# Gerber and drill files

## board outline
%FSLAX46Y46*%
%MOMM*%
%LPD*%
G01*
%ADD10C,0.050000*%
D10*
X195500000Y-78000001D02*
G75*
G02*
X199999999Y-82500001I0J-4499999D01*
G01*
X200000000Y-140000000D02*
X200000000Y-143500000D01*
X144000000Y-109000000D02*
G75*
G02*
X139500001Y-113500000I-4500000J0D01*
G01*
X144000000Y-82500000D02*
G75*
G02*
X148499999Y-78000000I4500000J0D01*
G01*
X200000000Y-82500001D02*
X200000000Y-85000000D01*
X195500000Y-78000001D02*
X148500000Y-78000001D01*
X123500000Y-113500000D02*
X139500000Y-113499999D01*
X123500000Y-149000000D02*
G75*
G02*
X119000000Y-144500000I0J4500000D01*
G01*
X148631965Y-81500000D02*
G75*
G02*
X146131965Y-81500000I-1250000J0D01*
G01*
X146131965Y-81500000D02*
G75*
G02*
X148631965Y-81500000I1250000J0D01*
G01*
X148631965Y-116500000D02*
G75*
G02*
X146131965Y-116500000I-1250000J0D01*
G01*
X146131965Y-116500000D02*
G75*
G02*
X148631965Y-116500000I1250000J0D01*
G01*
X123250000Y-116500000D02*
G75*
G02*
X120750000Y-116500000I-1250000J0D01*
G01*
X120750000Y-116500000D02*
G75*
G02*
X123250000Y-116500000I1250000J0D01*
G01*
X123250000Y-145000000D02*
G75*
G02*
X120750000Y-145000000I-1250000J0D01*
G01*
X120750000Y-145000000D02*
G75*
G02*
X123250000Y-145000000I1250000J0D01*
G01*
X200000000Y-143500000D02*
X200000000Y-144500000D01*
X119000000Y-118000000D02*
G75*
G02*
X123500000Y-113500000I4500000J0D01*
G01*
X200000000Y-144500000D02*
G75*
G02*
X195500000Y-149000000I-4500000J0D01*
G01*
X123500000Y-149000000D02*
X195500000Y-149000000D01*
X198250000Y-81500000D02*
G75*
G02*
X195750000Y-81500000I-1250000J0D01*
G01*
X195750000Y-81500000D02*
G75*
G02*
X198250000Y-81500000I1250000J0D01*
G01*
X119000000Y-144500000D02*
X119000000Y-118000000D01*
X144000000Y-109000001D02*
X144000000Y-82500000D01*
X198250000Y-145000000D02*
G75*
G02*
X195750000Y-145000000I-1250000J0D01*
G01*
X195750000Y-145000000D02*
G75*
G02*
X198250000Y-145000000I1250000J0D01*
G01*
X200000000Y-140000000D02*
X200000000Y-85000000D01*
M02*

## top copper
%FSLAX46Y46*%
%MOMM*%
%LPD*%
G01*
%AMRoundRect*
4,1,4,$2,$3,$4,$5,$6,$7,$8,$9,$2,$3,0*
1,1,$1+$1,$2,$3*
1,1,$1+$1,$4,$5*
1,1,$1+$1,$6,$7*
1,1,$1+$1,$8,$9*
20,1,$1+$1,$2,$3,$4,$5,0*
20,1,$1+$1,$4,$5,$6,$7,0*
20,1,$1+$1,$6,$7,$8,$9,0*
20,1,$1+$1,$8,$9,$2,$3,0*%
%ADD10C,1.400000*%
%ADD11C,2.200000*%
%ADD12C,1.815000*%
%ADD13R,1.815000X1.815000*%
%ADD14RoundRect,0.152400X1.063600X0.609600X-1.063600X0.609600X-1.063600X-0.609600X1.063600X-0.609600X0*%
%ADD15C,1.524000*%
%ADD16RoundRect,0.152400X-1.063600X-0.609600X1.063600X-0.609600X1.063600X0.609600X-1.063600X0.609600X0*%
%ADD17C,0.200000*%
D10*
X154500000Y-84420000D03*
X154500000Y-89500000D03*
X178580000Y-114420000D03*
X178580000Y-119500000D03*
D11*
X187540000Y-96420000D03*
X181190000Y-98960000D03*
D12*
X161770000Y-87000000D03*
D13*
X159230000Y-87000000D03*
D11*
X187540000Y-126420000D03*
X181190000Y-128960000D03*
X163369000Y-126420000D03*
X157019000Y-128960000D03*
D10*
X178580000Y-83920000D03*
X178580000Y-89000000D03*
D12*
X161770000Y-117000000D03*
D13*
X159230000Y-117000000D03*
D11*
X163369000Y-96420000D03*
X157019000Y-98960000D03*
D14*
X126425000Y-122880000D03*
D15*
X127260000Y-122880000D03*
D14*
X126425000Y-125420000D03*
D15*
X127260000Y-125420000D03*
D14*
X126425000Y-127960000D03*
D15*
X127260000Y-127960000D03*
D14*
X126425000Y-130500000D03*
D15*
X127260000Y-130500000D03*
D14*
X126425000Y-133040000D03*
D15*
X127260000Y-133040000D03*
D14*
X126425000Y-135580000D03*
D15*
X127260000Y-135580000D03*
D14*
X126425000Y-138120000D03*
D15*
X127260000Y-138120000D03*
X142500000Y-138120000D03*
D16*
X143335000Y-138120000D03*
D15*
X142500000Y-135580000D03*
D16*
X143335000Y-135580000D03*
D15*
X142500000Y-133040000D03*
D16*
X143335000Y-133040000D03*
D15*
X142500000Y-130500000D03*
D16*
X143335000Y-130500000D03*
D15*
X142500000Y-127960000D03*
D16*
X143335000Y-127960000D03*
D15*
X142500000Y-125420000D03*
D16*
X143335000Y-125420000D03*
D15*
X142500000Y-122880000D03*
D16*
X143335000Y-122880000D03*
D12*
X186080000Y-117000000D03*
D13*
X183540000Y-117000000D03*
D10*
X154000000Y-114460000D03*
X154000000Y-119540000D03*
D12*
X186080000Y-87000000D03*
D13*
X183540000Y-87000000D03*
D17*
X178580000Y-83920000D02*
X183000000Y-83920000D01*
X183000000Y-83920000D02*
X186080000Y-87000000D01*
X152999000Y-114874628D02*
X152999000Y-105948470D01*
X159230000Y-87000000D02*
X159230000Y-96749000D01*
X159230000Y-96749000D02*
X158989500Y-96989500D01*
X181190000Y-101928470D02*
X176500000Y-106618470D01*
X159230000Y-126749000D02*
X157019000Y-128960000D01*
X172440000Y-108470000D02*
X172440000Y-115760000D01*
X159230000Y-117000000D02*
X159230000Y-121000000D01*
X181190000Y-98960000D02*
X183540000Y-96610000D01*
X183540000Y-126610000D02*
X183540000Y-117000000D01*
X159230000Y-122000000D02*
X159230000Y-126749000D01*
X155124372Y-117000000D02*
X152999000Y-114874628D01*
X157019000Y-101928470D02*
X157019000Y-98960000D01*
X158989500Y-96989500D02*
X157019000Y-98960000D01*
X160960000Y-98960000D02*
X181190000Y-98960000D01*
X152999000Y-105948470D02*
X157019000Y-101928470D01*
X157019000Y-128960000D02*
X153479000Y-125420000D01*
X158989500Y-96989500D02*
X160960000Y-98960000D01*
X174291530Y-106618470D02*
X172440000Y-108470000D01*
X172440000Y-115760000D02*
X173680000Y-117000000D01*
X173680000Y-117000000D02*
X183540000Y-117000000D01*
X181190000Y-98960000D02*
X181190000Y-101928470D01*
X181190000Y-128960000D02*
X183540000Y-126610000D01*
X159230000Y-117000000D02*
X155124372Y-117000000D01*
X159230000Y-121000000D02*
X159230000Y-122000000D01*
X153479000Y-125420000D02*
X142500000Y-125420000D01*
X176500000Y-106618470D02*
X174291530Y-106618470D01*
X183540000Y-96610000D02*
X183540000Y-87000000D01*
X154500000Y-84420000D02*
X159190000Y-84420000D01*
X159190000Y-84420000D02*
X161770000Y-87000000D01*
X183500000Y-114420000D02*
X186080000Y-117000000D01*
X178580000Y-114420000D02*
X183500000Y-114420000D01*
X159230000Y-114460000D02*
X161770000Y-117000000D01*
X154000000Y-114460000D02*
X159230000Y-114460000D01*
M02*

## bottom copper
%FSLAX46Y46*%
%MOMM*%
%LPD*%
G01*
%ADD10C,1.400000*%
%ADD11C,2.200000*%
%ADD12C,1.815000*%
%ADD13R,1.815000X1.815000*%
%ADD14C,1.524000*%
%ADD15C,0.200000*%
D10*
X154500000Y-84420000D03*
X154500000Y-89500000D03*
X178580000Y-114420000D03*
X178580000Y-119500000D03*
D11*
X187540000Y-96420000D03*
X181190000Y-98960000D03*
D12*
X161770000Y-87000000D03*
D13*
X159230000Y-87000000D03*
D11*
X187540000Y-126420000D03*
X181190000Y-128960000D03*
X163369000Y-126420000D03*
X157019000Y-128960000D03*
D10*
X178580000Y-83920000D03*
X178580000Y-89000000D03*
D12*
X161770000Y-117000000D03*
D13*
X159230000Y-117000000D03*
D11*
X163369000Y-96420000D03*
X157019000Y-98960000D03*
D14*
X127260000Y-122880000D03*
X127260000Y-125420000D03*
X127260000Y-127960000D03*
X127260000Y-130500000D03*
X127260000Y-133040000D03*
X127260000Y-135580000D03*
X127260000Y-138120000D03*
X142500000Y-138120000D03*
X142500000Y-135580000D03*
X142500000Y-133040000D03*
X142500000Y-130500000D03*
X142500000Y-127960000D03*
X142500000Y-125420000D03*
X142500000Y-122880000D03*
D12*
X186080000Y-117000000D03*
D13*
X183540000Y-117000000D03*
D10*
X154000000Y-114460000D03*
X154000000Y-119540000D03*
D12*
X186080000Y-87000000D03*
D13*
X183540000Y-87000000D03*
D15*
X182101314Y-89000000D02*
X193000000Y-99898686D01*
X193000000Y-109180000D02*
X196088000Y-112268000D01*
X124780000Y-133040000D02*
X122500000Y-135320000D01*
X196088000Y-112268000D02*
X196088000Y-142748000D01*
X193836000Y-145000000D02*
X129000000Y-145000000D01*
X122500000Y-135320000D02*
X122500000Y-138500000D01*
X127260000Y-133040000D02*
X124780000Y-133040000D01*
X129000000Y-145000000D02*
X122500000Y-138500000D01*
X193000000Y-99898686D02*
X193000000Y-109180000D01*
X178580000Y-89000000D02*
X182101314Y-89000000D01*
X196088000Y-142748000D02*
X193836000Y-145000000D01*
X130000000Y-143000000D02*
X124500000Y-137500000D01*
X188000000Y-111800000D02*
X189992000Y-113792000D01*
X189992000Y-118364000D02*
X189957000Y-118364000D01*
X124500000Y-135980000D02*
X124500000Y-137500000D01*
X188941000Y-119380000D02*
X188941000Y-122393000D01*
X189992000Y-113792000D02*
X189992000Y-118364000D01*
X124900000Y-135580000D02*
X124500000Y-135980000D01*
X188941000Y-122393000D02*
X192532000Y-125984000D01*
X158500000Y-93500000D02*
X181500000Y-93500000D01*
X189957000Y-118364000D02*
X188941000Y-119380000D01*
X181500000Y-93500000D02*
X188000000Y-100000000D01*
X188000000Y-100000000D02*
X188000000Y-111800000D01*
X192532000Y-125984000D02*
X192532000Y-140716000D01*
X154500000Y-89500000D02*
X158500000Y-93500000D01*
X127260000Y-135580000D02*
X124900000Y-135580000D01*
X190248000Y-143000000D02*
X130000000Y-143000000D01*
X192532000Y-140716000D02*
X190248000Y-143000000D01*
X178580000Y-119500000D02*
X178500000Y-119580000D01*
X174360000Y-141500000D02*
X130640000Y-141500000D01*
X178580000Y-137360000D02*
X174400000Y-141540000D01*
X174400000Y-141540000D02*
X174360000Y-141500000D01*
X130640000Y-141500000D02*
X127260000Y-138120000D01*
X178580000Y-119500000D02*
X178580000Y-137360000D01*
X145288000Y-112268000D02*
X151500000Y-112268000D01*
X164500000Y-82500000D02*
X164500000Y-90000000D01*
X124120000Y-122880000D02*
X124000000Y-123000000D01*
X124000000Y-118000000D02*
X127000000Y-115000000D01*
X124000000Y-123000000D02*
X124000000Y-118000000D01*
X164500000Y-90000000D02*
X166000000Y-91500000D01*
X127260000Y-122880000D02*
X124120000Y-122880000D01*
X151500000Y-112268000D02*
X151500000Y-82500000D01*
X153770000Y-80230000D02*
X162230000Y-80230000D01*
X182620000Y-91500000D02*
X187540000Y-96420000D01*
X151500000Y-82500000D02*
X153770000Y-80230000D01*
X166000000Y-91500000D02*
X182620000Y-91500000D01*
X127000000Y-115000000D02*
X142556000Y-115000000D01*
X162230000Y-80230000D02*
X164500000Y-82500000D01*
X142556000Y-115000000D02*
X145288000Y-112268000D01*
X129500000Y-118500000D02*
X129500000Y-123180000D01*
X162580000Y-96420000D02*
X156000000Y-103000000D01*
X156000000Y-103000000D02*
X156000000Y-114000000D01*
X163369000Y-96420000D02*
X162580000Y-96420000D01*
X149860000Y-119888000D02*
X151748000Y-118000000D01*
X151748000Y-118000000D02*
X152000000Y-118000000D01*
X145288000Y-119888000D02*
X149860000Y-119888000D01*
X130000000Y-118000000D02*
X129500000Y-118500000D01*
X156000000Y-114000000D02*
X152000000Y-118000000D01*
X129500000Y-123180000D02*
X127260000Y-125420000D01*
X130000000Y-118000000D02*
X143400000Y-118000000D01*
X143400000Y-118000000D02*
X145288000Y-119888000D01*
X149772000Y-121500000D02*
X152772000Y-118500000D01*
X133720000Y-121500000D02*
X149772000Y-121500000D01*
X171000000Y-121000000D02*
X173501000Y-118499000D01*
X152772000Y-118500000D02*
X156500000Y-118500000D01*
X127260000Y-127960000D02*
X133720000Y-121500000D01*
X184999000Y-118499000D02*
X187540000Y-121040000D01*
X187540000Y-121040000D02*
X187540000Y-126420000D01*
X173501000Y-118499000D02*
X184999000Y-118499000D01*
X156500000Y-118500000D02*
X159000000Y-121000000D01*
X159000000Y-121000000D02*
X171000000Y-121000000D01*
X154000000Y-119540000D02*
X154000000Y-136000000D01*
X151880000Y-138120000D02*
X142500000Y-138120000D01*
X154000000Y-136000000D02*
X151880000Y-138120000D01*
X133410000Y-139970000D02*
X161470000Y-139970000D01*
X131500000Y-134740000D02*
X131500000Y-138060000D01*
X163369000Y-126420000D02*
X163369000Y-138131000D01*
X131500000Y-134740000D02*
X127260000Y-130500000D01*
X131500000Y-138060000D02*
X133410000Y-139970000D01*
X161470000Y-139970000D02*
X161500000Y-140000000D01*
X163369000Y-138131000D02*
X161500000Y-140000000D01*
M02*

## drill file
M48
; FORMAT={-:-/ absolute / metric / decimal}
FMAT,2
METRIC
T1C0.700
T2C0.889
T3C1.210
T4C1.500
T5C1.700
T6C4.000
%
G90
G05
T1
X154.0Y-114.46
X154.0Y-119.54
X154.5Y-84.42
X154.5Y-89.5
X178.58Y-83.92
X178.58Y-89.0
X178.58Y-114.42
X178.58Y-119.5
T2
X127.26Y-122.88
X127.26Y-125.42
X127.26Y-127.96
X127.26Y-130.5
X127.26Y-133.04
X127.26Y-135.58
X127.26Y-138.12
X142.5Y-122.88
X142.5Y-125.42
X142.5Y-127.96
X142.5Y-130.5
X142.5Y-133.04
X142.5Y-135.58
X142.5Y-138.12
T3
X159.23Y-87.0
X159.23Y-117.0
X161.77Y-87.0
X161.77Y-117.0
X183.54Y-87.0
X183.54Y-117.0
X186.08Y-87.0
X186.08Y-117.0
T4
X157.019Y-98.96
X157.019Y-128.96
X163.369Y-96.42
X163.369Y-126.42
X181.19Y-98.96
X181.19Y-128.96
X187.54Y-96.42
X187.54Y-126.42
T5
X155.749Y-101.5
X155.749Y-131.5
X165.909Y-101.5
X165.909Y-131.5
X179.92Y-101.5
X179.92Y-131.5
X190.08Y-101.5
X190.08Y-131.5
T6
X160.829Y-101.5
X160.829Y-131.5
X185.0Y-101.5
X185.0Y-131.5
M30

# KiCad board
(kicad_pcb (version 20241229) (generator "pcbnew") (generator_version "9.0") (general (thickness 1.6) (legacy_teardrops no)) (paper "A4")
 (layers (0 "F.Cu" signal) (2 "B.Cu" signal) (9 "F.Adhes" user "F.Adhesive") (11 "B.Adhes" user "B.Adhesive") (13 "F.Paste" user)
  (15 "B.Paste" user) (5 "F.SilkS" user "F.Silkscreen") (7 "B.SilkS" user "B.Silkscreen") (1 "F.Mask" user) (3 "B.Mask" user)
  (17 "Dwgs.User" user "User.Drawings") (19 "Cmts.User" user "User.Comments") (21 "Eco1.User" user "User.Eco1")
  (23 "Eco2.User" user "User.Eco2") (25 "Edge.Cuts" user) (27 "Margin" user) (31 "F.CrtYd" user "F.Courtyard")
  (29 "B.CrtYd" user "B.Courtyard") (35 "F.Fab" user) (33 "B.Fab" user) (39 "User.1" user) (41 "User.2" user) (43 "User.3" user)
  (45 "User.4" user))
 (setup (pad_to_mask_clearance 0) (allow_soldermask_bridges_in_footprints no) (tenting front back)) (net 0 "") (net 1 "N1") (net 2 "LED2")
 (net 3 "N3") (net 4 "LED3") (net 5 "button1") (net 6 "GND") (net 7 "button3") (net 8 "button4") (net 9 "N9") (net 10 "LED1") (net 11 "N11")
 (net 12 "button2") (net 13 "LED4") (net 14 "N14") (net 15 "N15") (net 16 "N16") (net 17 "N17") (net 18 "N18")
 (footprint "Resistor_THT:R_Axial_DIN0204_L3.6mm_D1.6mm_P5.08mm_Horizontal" (layer "F.Cu") (at 154.5 84.42 -90)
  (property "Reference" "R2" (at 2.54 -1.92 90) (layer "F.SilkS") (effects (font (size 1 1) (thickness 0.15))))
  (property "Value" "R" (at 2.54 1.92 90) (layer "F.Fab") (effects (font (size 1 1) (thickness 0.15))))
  (pad "1" thru_hole circle (at 0 0 270) (size 1.4 1.4) (drill 0.7) (layers "*.Cu" "*.Mask") (remove_unused_layers no) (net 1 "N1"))
  (pad "2" thru_hole circle (at 5.08 0 270) (size 1.4 1.4) (drill 0.7) (layers "*.Cu" "*.Mask") (remove_unused_layers no) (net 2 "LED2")))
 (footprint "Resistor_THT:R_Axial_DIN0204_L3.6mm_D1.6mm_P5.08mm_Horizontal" (layer "F.Cu") (at 178.58 114.42 -90)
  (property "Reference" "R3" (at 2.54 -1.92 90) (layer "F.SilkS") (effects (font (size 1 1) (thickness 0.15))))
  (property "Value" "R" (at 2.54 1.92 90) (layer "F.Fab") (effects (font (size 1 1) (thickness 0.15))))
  (pad "1" thru_hole circle (at 0 0 270) (size 1.4 1.4) (drill 0.7) (layers "*.Cu" "*.Mask") (remove_unused_layers no) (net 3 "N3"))
  (pad "2" thru_hole circle (at 5.08 0 270) (size 1.4 1.4) (drill 0.7) (layers "*.Cu" "*.Mask") (remove_unused_layers no) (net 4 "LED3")))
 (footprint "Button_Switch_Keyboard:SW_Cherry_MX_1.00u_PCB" (layer "F.Cu") (at 187.54 96.42)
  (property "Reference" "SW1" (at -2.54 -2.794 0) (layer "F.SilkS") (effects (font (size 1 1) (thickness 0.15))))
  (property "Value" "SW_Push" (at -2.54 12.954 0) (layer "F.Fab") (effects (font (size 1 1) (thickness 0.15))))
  (pad "" np_thru_hole circle (at -7.62 5.08) (size 1.7 1.7) (drill 1.7) (layers "*.Cu" "*.Mask"))
  (pad "" np_thru_hole circle (at -2.54 5.08) (size 4 4) (drill 4) (layers "*.Cu" "*.Mask"))
  (pad "" np_thru_hole circle (at 2.54 5.08) (size 1.7 1.7) (drill 1.7) (layers "*.Cu" "*.Mask"))
  (pad "1" thru_hole circle (at 0 0) (size 2.2 2.2) (drill 1.5) (layers "*.Cu" "*.Mask") (remove_unused_layers no) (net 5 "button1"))
  (pad "2" thru_hole circle (at -6.35 2.54) (size 2.2 2.2) (drill 1.5) (layers "*.Cu" "*.Mask") (remove_unused_layers no) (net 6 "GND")))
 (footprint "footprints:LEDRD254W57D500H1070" (layer "F.Cu") (at 160.5 87)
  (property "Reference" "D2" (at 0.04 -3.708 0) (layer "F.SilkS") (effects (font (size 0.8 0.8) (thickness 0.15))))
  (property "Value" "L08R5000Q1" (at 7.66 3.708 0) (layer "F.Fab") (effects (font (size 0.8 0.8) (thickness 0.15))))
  (pad "A" thru_hole circle (at 1.27 0) (size 1.815 1.815) (drill 1.21) (layers "*.Cu" "*.Mask") (remove_unused_layers no) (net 1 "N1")
   (solder_mask_margin 0.102))
  (pad "C" thru_hole rect (at -1.27 0) (size 1.815 1.815) (drill 1.21) (layers "*.Cu" "*.Mask") (remove_unused_layers no) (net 6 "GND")
   (solder_mask_margin 0.102)))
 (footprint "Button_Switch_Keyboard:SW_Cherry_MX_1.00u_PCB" (layer "F.Cu") (at 187.54 126.42)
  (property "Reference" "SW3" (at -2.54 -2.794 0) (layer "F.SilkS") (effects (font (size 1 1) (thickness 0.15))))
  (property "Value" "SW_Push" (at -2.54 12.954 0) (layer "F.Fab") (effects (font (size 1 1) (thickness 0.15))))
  (pad "" np_thru_hole circle (at -7.62 5.08) (size 1.7 1.7) (drill 1.7) (layers "*.Cu" "*.Mask"))
  (pad "" np_thru_hole circle (at -2.54 5.08) (size 4 4) (drill 4) (layers "*.Cu" "*.Mask"))
  (pad "" np_thru_hole circle (at 2.54 5.08) (size 1.7 1.7) (drill 1.7) (layers "*.Cu" "*.Mask"))
  (pad "1" thru_hole circle (at 0 0) (size 2.2 2.2) (drill 1.5) (layers "*.Cu" "*.Mask") (remove_unused_layers no) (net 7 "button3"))
  (pad "2" thru_hole circle (at -6.35 2.54) (size 2.2 2.2) (drill 1.5) (layers "*.Cu" "*.Mask") (remove_unused_layers no) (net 6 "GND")))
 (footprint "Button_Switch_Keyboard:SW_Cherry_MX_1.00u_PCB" (layer "F.Cu") (at 163.369 126.42)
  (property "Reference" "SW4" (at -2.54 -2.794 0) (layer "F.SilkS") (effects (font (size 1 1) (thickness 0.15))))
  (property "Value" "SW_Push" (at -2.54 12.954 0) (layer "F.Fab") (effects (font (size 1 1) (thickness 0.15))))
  (pad "" np_thru_hole circle (at -7.62 5.08) (size 1.7 1.7) (drill 1.7) (layers "*.Cu" "*.Mask"))
  (pad "" np_thru_hole circle (at -2.54 5.08) (size 4 4) (drill 4) (layers "*.Cu" "*.Mask"))
  (pad "" np_thru_hole circle (at 2.54 5.08) (size 1.7 1.7) (drill 1.7) (layers "*.Cu" "*.Mask"))
  (pad "1" thru_hole circle (at 0 0) (size 2.2 2.2) (drill 1.5) (layers "*.Cu" "*.Mask") (remove_unused_layers no) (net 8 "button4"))
  (pad "2" thru_hole circle (at -6.35 2.54) (size 2.2 2.2) (drill 1.5) (layers "*.Cu" "*.Mask") (remove_unused_layers no) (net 6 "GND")))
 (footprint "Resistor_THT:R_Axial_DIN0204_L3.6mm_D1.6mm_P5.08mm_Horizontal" (layer "F.Cu") (at 178.58 83.92 -90)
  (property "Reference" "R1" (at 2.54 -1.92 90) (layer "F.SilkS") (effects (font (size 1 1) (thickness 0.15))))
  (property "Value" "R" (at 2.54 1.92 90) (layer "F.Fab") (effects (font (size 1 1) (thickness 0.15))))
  (pad "1" thru_hole circle (at 0 0 270) (size 1.4 1.4) (drill 0.7) (layers "*.Cu" "*.Mask") (remove_unused_layers no) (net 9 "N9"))
  (pad "2" thru_hole circle (at 5.08 0 270) (size 1.4 1.4) (drill 0.7) (layers "*.Cu" "*.Mask") (remove_unused_layers no) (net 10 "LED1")))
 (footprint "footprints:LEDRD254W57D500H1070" (layer "F.Cu") (at 160.5 117)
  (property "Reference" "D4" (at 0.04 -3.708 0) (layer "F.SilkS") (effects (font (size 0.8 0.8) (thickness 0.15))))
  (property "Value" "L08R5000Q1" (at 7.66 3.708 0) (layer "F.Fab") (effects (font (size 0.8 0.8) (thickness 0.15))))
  (pad "A" thru_hole circle (at 1.27 0) (size 1.815 1.815) (drill 1.21) (layers "*.Cu" "*.Mask") (remove_unused_layers no) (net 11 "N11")
   (solder_mask_margin 0.102))
  (pad "C" thru_hole rect (at -1.27 0) (size 1.815 1.815) (drill 1.21) (layers "*.Cu" "*.Mask") (remove_unused_layers no) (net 6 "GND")
   (solder_mask_margin 0.102)))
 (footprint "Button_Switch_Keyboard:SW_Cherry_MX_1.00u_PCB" (layer "F.Cu") (at 163.369 96.42)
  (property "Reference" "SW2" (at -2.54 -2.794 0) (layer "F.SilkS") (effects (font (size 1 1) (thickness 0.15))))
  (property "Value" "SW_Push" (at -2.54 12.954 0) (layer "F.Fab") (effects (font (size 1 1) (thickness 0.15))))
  (pad "" np_thru_hole circle (at -7.62 5.08) (size 1.7 1.7) (drill 1.7) (layers "*.Cu" "*.Mask"))
  (pad "" np_thru_hole circle (at -2.54 5.08) (size 4 4) (drill 4) (layers "*.Cu" "*.Mask"))
  (pad "" np_thru_hole circle (at 2.54 5.08) (size 1.7 1.7) (drill 1.7) (layers "*.Cu" "*.Mask"))
  (pad "1" thru_hole circle (at 0 0) (size 2.2 2.2) (drill 1.5) (layers "*.Cu" "*.Mask") (remove_unused_layers no) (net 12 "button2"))
  (pad "2" thru_hole circle (at -6.35 2.54) (size 2.2 2.2) (drill 1.5) (layers "*.Cu" "*.Mask") (remove_unused_layers no) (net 6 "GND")))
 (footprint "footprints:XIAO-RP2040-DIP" (layer "F.Cu") (at 134.88 130.5)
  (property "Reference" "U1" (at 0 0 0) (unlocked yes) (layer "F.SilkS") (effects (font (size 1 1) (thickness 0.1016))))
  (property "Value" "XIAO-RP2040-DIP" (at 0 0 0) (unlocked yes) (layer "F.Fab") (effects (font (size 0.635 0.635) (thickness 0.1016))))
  (pad "1" smd roundrect (at -8.455 -7.62 180) (size 2.432 1.524) (layers "F.Cu" "F.Mask") (roundrect_rratio 0.1) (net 5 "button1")
   (thermal_bridge_angle 45))
  (pad "1" thru_hole circle (at -7.62 -7.62 180) (size 1.524 1.524) (drill 0.889) (layers "*.Cu" "*.Mask") (remove_unused_layers no)
   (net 5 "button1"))
  (pad "2" smd roundrect (at -8.455 -5.08 180) (size 2.432 1.524) (layers "F.Cu" "F.Mask") (roundrect_rratio 0.1) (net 12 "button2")
   (thermal_bridge_angle 45))
  (pad "2" thru_hole circle (at -7.62 -5.08 180) (size 1.524 1.524) (drill 0.889) (layers "*.Cu" "*.Mask") (remove_unused_layers no)
   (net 12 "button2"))
  (pad "3" smd roundrect (at -8.455 -2.54 180) (size 2.432 1.524) (layers "F.Cu" "F.Mask") (roundrect_rratio 0.1) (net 7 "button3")
   (thermal_bridge_angle 45))
  (pad "3" thru_hole circle (at -7.62 -2.54 180) (size 1.524 1.524) (drill 0.889) (layers "*.Cu" "*.Mask") (remove_unused_layers no)
   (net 7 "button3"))
  (pad "4" smd roundrect (at -8.455 0 180) (size 2.432 1.524) (layers "F.Cu" "F.Mask") (roundrect_rratio 0.1) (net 8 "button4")
   (thermal_bridge_angle 45))
  (pad "4" thru_hole circle (at -7.62 0 180) (size 1.524 1.524) (drill 0.889) (layers "*.Cu" "*.Mask") (remove_unused_layers no)
   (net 8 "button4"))
  (pad "5" smd roundrect (at -8.455 2.54 180) (size 2.432 1.524) (layers "F.Cu" "F.Mask") (roundrect_rratio 0.1) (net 10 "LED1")
   (thermal_bridge_angle 45))
  (pad "5" thru_hole circle (at -7.62 2.54 180) (size 1.524 1.524) (drill 0.889) (layers "*.Cu" "*.Mask") (remove_unused_layers no)
   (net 10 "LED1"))
  (pad "6" smd roundrect (at -8.455 5.08 180) (size 2.432 1.524) (layers "F.Cu" "F.Mask") (roundrect_rratio 0.1) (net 2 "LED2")
   (thermal_bridge_angle 45))
  (pad "6" thru_hole circle (at -7.62 5.08 180) (size 1.524 1.524) (drill 0.889) (layers "*.Cu" "*.Mask") (remove_unused_layers no)
   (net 2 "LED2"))
  (pad "7" smd roundrect (at -8.455 7.62 180) (size 2.432 1.524) (layers "F.Cu" "F.Mask") (roundrect_rratio 0.1) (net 4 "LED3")
   (thermal_bridge_angle 45))
  (pad "7" thru_hole circle (at -7.62 7.62 180) (size 1.524 1.524) (drill 0.889) (layers "*.Cu" "*.Mask") (remove_unused_layers no)
   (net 4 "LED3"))
  (pad "8" thru_hole circle (at 7.62 7.62) (size 1.524 1.524) (drill 0.889) (layers "*.Cu" "*.Mask") (remove_unused_layers no)
   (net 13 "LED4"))
  (pad "8" smd roundrect (at 8.455 7.62) (size 2.432 1.524) (layers "F.Cu" "F.Mask") (roundrect_rratio 0.1) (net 13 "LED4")
   (thermal_bridge_angle 45))
  (pad "9" thru_hole circle (at 7.62 5.08) (size 1.524 1.524) (drill 0.889) (layers "*.Cu" "*.Mask") (remove_unused_layers no)
   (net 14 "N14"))
  (pad "9" smd roundrect (at 8.455 5.08) (size 2.432 1.524) (layers "F.Cu" "F.Mask") (roundrect_rratio 0.1) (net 14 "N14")
   (thermal_bridge_angle 45))
  (pad "10" thru_hole circle (at 7.62 2.54) (size 1.524 1.524) (drill 0.889) (layers "*.Cu" "*.Mask") (remove_unused_layers no)
   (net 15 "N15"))
  (pad "10" smd roundrect (at 8.455 2.54) (size 2.432 1.524) (layers "F.Cu" "F.Mask") (roundrect_rratio 0.1) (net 15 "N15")
   (thermal_bridge_angle 45))
  (pad "11" thru_hole circle (at 7.62 0) (size 1.524 1.524) (drill 0.889) (layers "*.Cu" "*.Mask") (remove_unused_layers no) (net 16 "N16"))
  (pad "11" smd roundrect (at 8.455 0) (size 2.432 1.524) (layers "F.Cu" "F.Mask") (roundrect_rratio 0.1) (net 16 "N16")
   (thermal_bridge_angle 45))
  (pad "12" thru_hole circle (at 7.62 -2.54) (size 1.524 1.524) (drill 0.889) (layers "*.Cu" "*.Mask") (remove_unused_layers no)
   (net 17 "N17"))
  (pad "12" smd roundrect (at 8.455 -2.54) (size 2.432 1.524) (layers "F.Cu" "F.Mask") (roundrect_rratio 0.1) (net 17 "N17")
   (thermal_bridge_angle 45))
  (pad "13" thru_hole circle (at 7.62 -5.08) (size 1.524 1.524) (drill 0.889) (layers "*.Cu" "*.Mask") (remove_unused_layers no)
   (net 6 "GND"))
  (pad "13" smd roundrect (at 8.455 -5.08) (size 2.432 1.524) (layers "F.Cu" "F.Mask") (roundrect_rratio 0.1) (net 6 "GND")
   (thermal_bridge_angle 45))
  (pad "14" thru_hole circle (at 7.62 -7.62) (size 1.524 1.524) (drill 0.889) (layers "*.Cu" "*.Mask") (remove_unused_layers no)
   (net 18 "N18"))
  (pad "14" smd roundrect (at 8.455 -7.62) (size 2.432 1.524) (layers "F.Cu" "F.Mask") (roundrect_rratio 0.1) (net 18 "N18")
   (thermal_bridge_angle 45)))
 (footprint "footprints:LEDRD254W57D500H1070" (layer "F.Cu") (at 184.81 117)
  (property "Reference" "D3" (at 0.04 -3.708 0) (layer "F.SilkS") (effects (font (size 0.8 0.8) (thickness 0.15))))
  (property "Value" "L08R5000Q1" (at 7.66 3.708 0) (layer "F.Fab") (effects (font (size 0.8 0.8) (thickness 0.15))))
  (pad "A" thru_hole circle (at 1.27 0) (size 1.815 1.815) (drill 1.21) (layers "*.Cu" "*.Mask") (remove_unused_layers no) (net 3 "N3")
   (solder_mask_margin 0.102))
  (pad "C" thru_hole rect (at -1.27 0) (size 1.815 1.815) (drill 1.21) (layers "*.Cu" "*.Mask") (remove_unused_layers no) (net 6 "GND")
   (solder_mask_margin 0.102)))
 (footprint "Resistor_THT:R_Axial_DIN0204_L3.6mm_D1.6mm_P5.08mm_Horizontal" (layer "F.Cu") (at 154 114.46 -90)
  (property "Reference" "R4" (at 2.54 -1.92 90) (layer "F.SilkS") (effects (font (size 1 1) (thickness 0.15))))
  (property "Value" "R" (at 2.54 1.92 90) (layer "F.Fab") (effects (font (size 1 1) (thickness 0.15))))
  (pad "1" thru_hole circle (at 0 0 270) (size 1.4 1.4) (drill 0.7) (layers "*.Cu" "*.Mask") (remove_unused_layers no) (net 11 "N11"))
  (pad "2" thru_hole circle (at 5.08 0 270) (size 1.4 1.4) (drill 0.7) (layers "*.Cu" "*.Mask") (remove_unused_layers no) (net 13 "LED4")))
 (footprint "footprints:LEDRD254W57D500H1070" (layer "F.Cu") (at 184.81 87)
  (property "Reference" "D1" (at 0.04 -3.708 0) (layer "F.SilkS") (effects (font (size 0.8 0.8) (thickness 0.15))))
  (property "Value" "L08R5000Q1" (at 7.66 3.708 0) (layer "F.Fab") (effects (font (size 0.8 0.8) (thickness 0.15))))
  (pad "A" thru_hole circle (at 1.27 0) (size 1.815 1.815) (drill 1.21) (layers "*.Cu" "*.Mask") (remove_unused_layers no) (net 9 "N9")
   (solder_mask_margin 0.102))
  (pad "C" thru_hole rect (at -1.27 0) (size 1.815 1.815) (drill 1.21) (layers "*.Cu" "*.Mask") (remove_unused_layers no) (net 6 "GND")
   (solder_mask_margin 0.102)))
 (gr_arc (start 195.5 78.000001) (mid 198.681981 79.31802) (end 200 82.500001) (stroke (width 0.05) (type default)) (layer "Edge.Cuts"))
 (gr_line (start 200 140) (end 200 143.5) (stroke (width 0.05) (type default)) (layer "Edge.Cuts"))
 (gr_arc (start 144 109) (mid 142.681982 112.181986) (end 139.500001 113.499999) (stroke (width 0.05) (type default)) (layer "Edge.Cuts"))
 (gr_arc (start 144 82.5) (mid 145.31802 79.318026) (end 148.499999 78.000001) (stroke (width 0.05) (type default)) (layer "Edge.Cuts"))
 (gr_line (start 200 82.500001) (end 200 85) (stroke (width 0.05) (type default)) (layer "Edge.Cuts"))
 (gr_line (start 195.5 78.000001) (end 148.5 78.000001) (stroke (width 0.05) (type default)) (layer "Edge.Cuts"))
 (gr_line (start 123.5 113.5) (end 139.5 113.499999) (stroke (width 0.05) (type default)) (layer "Edge.Cuts"))
 (gr_arc (start 123.5 149) (mid 120.318019 147.681981) (end 119 144.5) (stroke (width 0.05) (type default)) (layer "Edge.Cuts"))
 (gr_circle (center 147.381965 81.5) (end 148.631965 81.5) (stroke (width 0.05) (type solid)) (fill no) (layer "Edge.Cuts"))
 (gr_circle (center 147.381965 116.5) (end 148.631965 116.5) (stroke (width 0.05) (type solid)) (fill no) (layer "Edge.Cuts"))
 (gr_circle (center 122 116.5) (end 123.25 116.5) (stroke (width 0.05) (type solid)) (fill no) (layer "Edge.Cuts"))
 (gr_circle (center 122 145) (end 123.25 145) (stroke (width 0.05) (type solid)) (fill no) (layer "Edge.Cuts"))
 (gr_line (start 200 143.5) (end 200 144.5) (stroke (width 0.05) (type default)) (layer "Edge.Cuts"))
 (gr_arc (start 119 118) (mid 120.31802 114.81802) (end 123.5 113.5) (stroke (width 0.05) (type default)) (layer "Edge.Cuts"))
 (gr_arc (start 200 144.5) (mid 198.681981 147.681981) (end 195.5 149) (stroke (width 0.05) (type default)) (layer "Edge.Cuts"))
 (gr_line (start 123.5 149) (end 195.5 149) (stroke (width 0.05) (type default)) (layer "Edge.Cuts"))
 (gr_circle (center 197 81.5) (end 198.25 81.5) (stroke (width 0.05) (type solid)) (fill no) (layer "Edge.Cuts"))
 (gr_line (start 119 144.5) (end 119 118) (stroke (width 0.05) (type default)) (layer "Edge.Cuts"))
 (gr_line (start 144 109.000001) (end 144 82.5) (stroke (width 0.05) (type default)) (layer "Edge.Cuts"))
 (gr_circle (center 197 145) (end 198.25 145) (stroke (width 0.05) (type solid)) (fill no) (layer "Edge.Cuts"))
 (gr_line (start 200 140) (end 200 85) (stroke (width 0.05) (type solid)) (layer "Edge.Cuts"))
 (segment (start 178.58 83.92) (end 183 83.92) (width 0.2) (layer "F.Cu") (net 9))
 (segment (start 183 83.92) (end 186.08 87) (width 0.2) (layer "F.Cu") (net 9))
 (segment (start 152.999 114.874628) (end 152.999 105.94847) (width 0.2) (layer "F.Cu") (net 6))
 (segment (start 159.23 87) (end 159.23 96.749) (width 0.2) (layer "F.Cu") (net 6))
 (segment (start 159.23 96.749) (end 158.9895 96.9895) (width 0.2) (layer "F.Cu") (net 6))
 (segment (start 181.19 101.92847) (end 176.5 106.61847) (width 0.2) (layer "F.Cu") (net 6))
 (segment (start 159.23 126.749) (end 157.019 128.96) (width 0.2) (layer "F.Cu") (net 6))
 (segment (start 172.44 108.47) (end 172.44 115.76) (width 0.2) (layer "F.Cu") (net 6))
 (segment (start 159.23 117) (end 159.23 121) (width 0.2) (layer "F.Cu") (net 6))
 (segment (start 181.19 98.96) (end 183.54 96.61) (width 0.2) (layer "F.Cu") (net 6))
 (segment (start 183.54 126.61) (end 183.54 117) (width 0.2) (layer "F.Cu") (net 6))
 (segment (start 159.23 122) (end 159.23 126.749) (width 0.2) (layer "F.Cu") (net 6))
 (segment (start 155.124372 117) (end 152.999 114.874628) (width 0.2) (layer "F.Cu") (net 6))
 (segment (start 157.019 101.92847) (end 157.019 98.96) (width 0.2) (layer "F.Cu") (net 6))
 (segment (start 158.9895 96.9895) (end 157.019 98.96) (width 0.2) (layer "F.Cu") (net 6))
 (segment (start 160.96 98.96) (end 181.19 98.96) (width 0.2) (layer "F.Cu") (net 6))
 (segment (start 152.999 105.94847) (end 157.019 101.92847) (width 0.2) (layer "F.Cu") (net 6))
 (segment (start 157.019 128.96) (end 153.479 125.42) (width 0.2) (layer "F.Cu") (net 6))
 (segment (start 158.9895 96.9895) (end 160.96 98.96) (width 0.2) (layer "F.Cu") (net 6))
 (segment (start 174.29153 106.61847) (end 172.44 108.47) (width 0.2) (layer "F.Cu") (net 6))
 (segment (start 172.44 115.76) (end 173.68 117) (width 0.2) (layer "F.Cu") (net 6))
 (segment (start 173.68 117) (end 183.54 117) (width 0.2) (layer "F.Cu") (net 6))
 (segment (start 181.19 98.96) (end 181.19 101.92847) (width 0.2) (layer "F.Cu") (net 6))
 (segment (start 181.19 128.96) (end 183.54 126.61) (width 0.2) (layer "F.Cu") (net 6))
 (segment (start 159.23 117) (end 155.124372 117) (width 0.2) (layer "F.Cu") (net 6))
 (segment (start 159.23 121) (end 159.23 122) (width 0.2) (layer "F.Cu") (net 6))
 (segment (start 153.479 125.42) (end 142.5 125.42) (width 0.2) (layer "F.Cu") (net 6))
 (segment (start 176.5 106.61847) (end 174.29153 106.61847) (width 0.2) (layer "F.Cu") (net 6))
 (segment (start 183.54 96.61) (end 183.54 87) (width 0.2) (layer "F.Cu") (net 6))
 (segment (start 154.5 84.42) (end 159.19 84.42) (width 0.2) (layer "F.Cu") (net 1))
 (segment (start 159.19 84.42) (end 161.77 87) (width 0.2) (layer "F.Cu") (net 1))
 (segment (start 183.5 114.42) (end 186.08 117) (width 0.2) (layer "F.Cu") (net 3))
 (segment (start 178.58 114.42) (end 183.5 114.42) (width 0.2) (layer "F.Cu") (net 3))
 (segment (start 182.101314 89) (end 193 99.898686) (width 0.2) (layer "B.Cu") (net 10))
 (segment (start 193 109.18) (end 196.088 112.268) (width 0.2) (layer "B.Cu") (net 10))
 (segment (start 124.78 133.04) (end 122.5 135.32) (width 0.2) (layer "B.Cu") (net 10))
 (segment (start 196.088 112.268) (end 196.088 142.748) (width 0.2) (layer "B.Cu") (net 10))
 (segment (start 193.836 145) (end 129 145) (width 0.2) (layer "B.Cu") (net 10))
 (segment (start 122.5 135.32) (end 122.5 138.5) (width 0.2) (layer "B.Cu") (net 10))
 (segment (start 127.26 133.04) (end 124.78 133.04) (width 0.2) (layer "B.Cu") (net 10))
 (segment (start 129 145) (end 122.5 138.5) (width 0.2) (layer "B.Cu") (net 10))
 (segment (start 193 99.898686) (end 193 109.18) (width 0.2) (layer "B.Cu") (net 10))
 (segment (start 178.58 89) (end 182.101314 89) (width 0.2) (layer "B.Cu") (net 10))
 (segment (start 196.088 142.748) (end 193.836 145) (width 0.2) (layer "B.Cu") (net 10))
 (segment (start 130 143) (end 124.5 137.5) (width 0.2) (layer "B.Cu") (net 2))
 (segment (start 188 111.8) (end 189.992 113.792) (width 0.2) (layer "B.Cu") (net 2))
 (segment (start 189.992 118.364) (end 189.957 118.364) (width 0.2) (layer "B.Cu") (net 2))
 (segment (start 124.5 135.98) (end 124.5 137.5) (width 0.2) (layer "B.Cu") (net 2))
 (segment (start 188.941 119.38) (end 188.941 122.393) (width 0.2) (layer "B.Cu") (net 2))
 (segment (start 189.992 113.792) (end 189.992 118.364) (width 0.2) (layer "B.Cu") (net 2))
 (segment (start 124.9 135.58) (end 124.5 135.98) (width 0.2) (layer "B.Cu") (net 2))
 (segment (start 188.941 122.393) (end 192.532 125.984) (width 0.2) (layer "B.Cu") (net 2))
 (segment (start 158.5 93.5) (end 181.5 93.5) (width 0.2) (layer "B.Cu") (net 2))
 (segment (start 189.957 118.364) (end 188.941 119.38) (width 0.2) (layer "B.Cu") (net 2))
 (segment (start 181.5 93.5) (end 188 100) (width 0.2) (layer "B.Cu") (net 2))
 (segment (start 188 100) (end 188 111.8) (width 0.2) (layer "B.Cu") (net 2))
 (segment (start 192.532 125.984) (end 192.532 140.716) (width 0.2) (layer "B.Cu") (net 2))
 (segment (start 154.5 89.5) (end 158.5 93.5) (width 0.2) (layer "B.Cu") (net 2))
 (segment (start 127.26 135.58) (end 124.9 135.58) (width 0.2) (layer "B.Cu") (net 2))
 (segment (start 190.248 143) (end 130 143) (width 0.2) (layer "B.Cu") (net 2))
 (segment (start 192.532 140.716) (end 190.248 143) (width 0.2) (layer "B.Cu") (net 2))
 (segment (start 178.58 119.5) (end 178.5 119.58) (width 0.2) (layer "B.Cu") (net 4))
 (segment (start 174.36 141.5) (end 130.64 141.5) (width 0.2) (layer "B.Cu") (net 4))
 (segment (start 178.58 137.36) (end 174.4 141.54) (width 0.2) (layer "B.Cu") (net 4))
 (segment (start 174.4 141.54) (end 174.36 141.5) (width 0.2) (layer "B.Cu") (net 4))
 (segment (start 130.64 141.5) (end 127.26 138.12) (width 0.2) (layer "B.Cu") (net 4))
 (segment (start 178.58 119.5) (end 178.58 137.36) (width 0.2) (layer "B.Cu") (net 4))
 (segment (start 145.288 112.268) (end 151.5 112.268) (width 0.2) (layer "B.Cu") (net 5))
 (segment (start 164.5 82.5) (end 164.5 90) (width 0.2) (layer "B.Cu") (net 5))
 (segment (start 124.12 122.88) (end 124 123) (width 0.2) (layer "B.Cu") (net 5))
 (segment (start 124 118) (end 127 115) (width 0.2) (layer "B.Cu") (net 5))
 (segment (start 124 123) (end 124 118) (width 0.2) (layer "B.Cu") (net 5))
 (segment (start 164.5 90) (end 166 91.5) (width 0.2) (layer "B.Cu") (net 5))
 (segment (start 127.26 122.88) (end 124.12 122.88) (width 0.2) (layer "B.Cu") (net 5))
 (segment (start 151.5 112.268) (end 151.5 82.5) (width 0.2) (layer "B.Cu") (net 5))
 (segment (start 153.77 80.23) (end 162.23 80.23) (width 0.2) (layer "B.Cu") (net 5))
 (segment (start 182.62 91.5) (end 187.54 96.42) (width 0.2) (layer "B.Cu") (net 5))
 (segment (start 151.5 82.5) (end 153.77 80.23) (width 0.2) (layer "B.Cu") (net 5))
 (segment (start 166 91.5) (end 182.62 91.5) (width 0.2) (layer "B.Cu") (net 5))
 (segment (start 127 115) (end 142.556 115) (width 0.2) (layer "B.Cu") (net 5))
 (segment (start 162.23 80.23) (end 164.5 82.5) (width 0.2) (layer "B.Cu") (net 5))
 (segment (start 142.556 115) (end 145.288 112.268) (width 0.2) (layer "B.Cu") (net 5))
 (segment (start 129.5 118.5) (end 129.5 123.18) (width 0.2) (layer "B.Cu") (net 12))
 (segment (start 162.58 96.42) (end 156 103) (width 0.2) (layer "B.Cu") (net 12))
 (segment (start 156 103) (end 156 114) (width 0.2) (layer "B.Cu") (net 12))
 (segment (start 163.369 96.42) (end 162.58 96.42) (width 0.2) (layer "B.Cu") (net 12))
 (segment (start 149.86 119.888) (end 151.748 118) (width 0.2) (layer "B.Cu") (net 12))
 (segment (start 151.748 118) (end 152 118) (width 0.2) (layer "B.Cu") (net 12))
 (segment (start 145.288 119.888) (end 149.86 119.888) (width 0.2) (layer "B.Cu") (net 12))
 (segment (start 130 118) (end 129.5 118.5) (width 0.2) (layer "B.Cu") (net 12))
 (segment (start 156 114) (end 152 118) (width 0.2) (layer "B.Cu") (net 12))
 (segment (start 129.5 123.18) (end 127.26 125.42) (width 0.2) (layer "B.Cu") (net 12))
 (segment (start 130 118) (end 143.4 118) (width 0.2) (layer "B.Cu") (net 12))
 (segment (start 143.4 118) (end 145.288 119.888) (width 0.2) (layer "B.Cu") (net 12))
 (segment (start 149.772 121.5) (end 152.772 118.5) (width 0.2) (layer "B.Cu") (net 7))
 (segment (start 133.72 121.5) (end 149.772 121.5) (width 0.2) (layer "B.Cu") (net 7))
 (segment (start 171 121) (end 173.501 118.499) (width 0.2) (layer "B.Cu") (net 7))
 (segment (start 152.772 118.5) (end 156.5 118.5) (width 0.2) (layer "B.Cu") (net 7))
 (segment (start 127.26 127.96) (end 133.72 121.5) (width 0.2) (layer "B.Cu") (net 7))
 (segment (start 184.999 118.499) (end 187.54 121.04) (width 0.2) (layer "B.Cu") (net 7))
 (segment (start 187.54 121.04) (end 187.54 126.42) (width 0.2) (layer "B.Cu") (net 7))
 (segment (start 173.501 118.499) (end 184.999 118.499) (width 0.2) (layer "B.Cu") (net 7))
 (segment (start 156.5 118.5) (end 159 121) (width 0.2) (layer "B.Cu") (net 7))
 (segment (start 159 121) (end 171 121) (width 0.2) (layer "B.Cu") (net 7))
 (segment (start 159.23 114.46) (end 161.77 117) (width 0.2) (layer "F.Cu") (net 11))
 (segment (start 154 114.46) (end 159.23 114.46) (width 0.2) (layer "F.Cu") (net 11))
 (segment (start 154 119.54) (end 154 136) (width 0.2) (layer "B.Cu") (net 13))
 (segment (start 151.88 138.12) (end 142.5 138.12) (width 0.2) (layer "B.Cu") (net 13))
 (segment (start 154 136) (end 151.88 138.12) (width 0.2) (layer "B.Cu") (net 13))
 (segment (start 133.41 139.97) (end 161.47 139.97) (width 0.2) (layer "B.Cu") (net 8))
 (segment (start 131.5 134.74) (end 131.5 138.06) (width 0.2) (layer "B.Cu") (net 8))
 (segment (start 163.369 126.42) (end 163.369 138.131) (width 0.2) (layer "B.Cu") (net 8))
 (segment (start 131.5 134.74) (end 127.26 130.5) (width 0.2) (layer "B.Cu") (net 8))
 (segment (start 131.5 138.06) (end 133.41 139.97) (width 0.2) (layer "B.Cu") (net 8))
 (segment (start 161.47 139.97) (end 161.5 140) (width 0.2) (layer "B.Cu") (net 8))
 (segment (start 163.369 138.131) (end 161.5 140) (width 0.2) (layer "B.Cu") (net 8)))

